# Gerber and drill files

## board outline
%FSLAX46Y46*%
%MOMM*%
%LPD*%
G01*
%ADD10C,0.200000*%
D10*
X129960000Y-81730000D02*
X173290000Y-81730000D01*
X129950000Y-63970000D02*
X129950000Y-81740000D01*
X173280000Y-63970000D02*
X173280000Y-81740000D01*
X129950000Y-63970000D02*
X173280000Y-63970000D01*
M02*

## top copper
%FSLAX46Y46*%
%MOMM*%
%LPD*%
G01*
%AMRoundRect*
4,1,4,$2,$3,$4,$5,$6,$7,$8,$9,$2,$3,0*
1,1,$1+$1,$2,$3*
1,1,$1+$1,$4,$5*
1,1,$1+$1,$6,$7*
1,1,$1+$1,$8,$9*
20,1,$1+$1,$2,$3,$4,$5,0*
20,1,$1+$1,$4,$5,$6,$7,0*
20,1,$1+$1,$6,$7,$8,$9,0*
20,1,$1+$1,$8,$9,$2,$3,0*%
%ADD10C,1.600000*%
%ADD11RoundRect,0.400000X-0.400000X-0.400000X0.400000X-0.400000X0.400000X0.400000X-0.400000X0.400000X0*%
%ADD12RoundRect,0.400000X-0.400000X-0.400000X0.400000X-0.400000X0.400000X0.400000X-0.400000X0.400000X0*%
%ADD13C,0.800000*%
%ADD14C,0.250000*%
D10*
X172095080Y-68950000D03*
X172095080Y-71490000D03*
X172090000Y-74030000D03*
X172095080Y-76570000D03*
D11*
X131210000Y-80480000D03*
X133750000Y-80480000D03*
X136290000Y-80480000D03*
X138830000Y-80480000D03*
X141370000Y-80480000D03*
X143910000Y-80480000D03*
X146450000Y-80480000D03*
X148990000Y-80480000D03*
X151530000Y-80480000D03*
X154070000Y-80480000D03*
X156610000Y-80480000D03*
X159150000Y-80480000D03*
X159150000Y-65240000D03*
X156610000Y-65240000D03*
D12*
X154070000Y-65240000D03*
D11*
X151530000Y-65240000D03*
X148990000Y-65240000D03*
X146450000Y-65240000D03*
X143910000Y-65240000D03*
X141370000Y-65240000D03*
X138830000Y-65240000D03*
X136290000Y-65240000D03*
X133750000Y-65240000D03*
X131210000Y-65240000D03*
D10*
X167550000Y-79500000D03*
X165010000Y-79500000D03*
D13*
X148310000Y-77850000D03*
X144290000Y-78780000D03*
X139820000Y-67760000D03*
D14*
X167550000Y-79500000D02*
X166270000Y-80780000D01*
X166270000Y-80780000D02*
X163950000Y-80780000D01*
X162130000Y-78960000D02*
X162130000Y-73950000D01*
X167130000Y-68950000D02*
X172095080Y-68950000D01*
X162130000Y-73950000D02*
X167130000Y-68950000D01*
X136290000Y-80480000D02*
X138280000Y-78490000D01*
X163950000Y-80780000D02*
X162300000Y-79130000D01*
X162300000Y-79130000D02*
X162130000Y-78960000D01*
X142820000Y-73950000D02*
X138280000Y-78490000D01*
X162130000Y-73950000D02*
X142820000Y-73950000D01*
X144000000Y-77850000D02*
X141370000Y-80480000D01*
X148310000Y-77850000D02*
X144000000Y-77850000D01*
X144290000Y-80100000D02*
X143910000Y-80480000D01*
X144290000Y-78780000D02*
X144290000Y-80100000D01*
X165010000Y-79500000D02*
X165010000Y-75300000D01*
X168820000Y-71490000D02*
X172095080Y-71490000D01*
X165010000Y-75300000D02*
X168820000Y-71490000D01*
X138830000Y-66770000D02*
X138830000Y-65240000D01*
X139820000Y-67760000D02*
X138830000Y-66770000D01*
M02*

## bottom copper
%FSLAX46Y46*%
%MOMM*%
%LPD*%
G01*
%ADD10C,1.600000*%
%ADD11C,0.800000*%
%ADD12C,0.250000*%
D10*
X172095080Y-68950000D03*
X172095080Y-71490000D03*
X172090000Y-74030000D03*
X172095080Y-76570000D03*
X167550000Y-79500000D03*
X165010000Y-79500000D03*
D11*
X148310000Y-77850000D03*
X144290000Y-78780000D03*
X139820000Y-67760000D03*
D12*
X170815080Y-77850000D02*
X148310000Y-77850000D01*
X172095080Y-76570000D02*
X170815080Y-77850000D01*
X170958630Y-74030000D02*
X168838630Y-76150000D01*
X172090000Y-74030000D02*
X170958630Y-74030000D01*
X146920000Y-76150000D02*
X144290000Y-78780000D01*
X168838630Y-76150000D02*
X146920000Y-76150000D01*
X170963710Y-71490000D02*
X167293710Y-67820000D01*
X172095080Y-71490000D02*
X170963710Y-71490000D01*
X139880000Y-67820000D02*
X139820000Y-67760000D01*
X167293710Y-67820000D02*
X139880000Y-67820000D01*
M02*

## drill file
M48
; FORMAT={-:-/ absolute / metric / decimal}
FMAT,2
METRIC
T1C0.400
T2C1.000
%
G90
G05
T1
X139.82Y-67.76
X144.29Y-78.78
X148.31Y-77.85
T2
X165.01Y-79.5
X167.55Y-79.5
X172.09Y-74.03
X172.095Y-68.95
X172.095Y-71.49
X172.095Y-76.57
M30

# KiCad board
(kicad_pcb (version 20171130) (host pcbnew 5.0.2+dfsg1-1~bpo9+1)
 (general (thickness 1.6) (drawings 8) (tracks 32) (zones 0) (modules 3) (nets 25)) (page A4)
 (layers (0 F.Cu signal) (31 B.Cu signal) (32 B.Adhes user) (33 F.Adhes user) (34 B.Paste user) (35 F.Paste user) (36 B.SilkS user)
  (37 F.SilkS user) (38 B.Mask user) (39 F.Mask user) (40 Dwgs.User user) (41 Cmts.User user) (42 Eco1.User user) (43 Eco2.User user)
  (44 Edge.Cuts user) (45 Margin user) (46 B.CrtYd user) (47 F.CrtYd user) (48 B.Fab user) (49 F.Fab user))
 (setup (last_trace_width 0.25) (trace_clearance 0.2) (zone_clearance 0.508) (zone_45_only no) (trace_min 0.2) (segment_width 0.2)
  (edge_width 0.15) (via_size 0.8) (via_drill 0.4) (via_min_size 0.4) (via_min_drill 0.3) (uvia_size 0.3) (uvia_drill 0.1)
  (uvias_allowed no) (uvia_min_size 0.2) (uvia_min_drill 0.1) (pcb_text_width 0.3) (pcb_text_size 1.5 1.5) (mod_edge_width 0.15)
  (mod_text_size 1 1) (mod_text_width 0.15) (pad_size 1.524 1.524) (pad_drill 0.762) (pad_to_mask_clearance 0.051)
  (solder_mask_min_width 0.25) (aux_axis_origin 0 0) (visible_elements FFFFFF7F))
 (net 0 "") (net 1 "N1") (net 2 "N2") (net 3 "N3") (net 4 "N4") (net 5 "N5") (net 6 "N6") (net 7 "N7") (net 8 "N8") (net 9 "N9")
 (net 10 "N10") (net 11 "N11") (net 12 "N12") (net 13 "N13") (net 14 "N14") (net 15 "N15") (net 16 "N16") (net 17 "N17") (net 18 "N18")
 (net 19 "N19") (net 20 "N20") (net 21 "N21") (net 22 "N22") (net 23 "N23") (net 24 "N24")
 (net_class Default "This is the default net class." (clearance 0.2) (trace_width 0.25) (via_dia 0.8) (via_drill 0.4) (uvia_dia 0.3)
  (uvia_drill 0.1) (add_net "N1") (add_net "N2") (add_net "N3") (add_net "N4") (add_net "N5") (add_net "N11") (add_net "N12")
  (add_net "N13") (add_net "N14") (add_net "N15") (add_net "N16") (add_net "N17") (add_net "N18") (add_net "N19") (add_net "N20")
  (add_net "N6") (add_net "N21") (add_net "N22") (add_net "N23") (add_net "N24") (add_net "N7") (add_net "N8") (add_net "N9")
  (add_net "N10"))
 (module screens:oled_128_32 (layer F.Cu) (at 172.09508 72.76 270)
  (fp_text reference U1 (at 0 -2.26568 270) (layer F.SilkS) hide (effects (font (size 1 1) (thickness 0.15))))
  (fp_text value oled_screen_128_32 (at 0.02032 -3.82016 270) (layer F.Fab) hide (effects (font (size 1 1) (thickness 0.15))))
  (pad 1 thru_hole circle (at -3.81 0 270) (size 1.6 1.6) (drill 1) (layers *.Cu *.Mask) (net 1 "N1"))
  (pad 2 thru_hole circle (at -1.27 0 270) (size 1.6 1.6) (drill 1) (layers *.Cu *.Mask) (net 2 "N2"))
  (pad 3 thru_hole circle (at 1.27 0.00508 270) (size 1.6 1.6) (drill 1) (layers *.Cu *.Mask) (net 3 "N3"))
  (pad 4 thru_hole circle (at 3.81 0 270) (size 1.6 1.6) (drill 1) (layers *.Cu *.Mask) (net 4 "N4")))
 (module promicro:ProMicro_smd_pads (layer F.Cu) (at 145.18 72.86)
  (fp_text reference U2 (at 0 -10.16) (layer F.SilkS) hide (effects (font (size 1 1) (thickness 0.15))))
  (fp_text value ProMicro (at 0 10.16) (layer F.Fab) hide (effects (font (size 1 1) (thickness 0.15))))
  (pad 1 smd roundrect (at -13.97 7.62) (size 1.6 1.6) (layers F.Cu F.Paste F.Mask) (roundrect_rratio 0.25) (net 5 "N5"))
  (pad 2 smd roundrect (at -11.43 7.62) (size 1.6 1.6) (layers F.Cu F.Paste F.Mask) (roundrect_rratio 0.25) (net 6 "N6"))
  (pad 3 smd roundrect (at -8.89 7.62) (size 1.6 1.6) (layers F.Cu F.Paste F.Mask) (roundrect_rratio 0.25) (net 1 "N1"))
  (pad 4 smd roundrect (at -6.35 7.62) (size 1.6 1.6) (layers F.Cu F.Paste F.Mask) (roundrect_rratio 0.25) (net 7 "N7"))
  (pad 5 smd roundrect (at -3.81 7.62) (size 1.6 1.6) (layers F.Cu F.Paste F.Mask) (roundrect_rratio 0.25) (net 4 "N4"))
  (pad 6 smd roundrect (at -1.27 7.62) (size 1.6 1.6) (layers F.Cu F.Paste F.Mask) (roundrect_rratio 0.25) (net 3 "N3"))
  (pad 7 smd roundrect (at 1.27 7.62) (size 1.6 1.6) (layers F.Cu F.Paste F.Mask) (roundrect_rratio 0.25) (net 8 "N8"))
  (pad 8 smd roundrect (at 3.81 7.62) (size 1.6 1.6) (layers F.Cu F.Paste F.Mask) (roundrect_rratio 0.25) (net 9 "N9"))
  (pad 9 smd roundrect (at 6.35 7.62) (size 1.6 1.6) (layers F.Cu F.Paste F.Mask) (roundrect_rratio 0.25) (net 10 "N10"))
  (pad 10 smd roundrect (at 8.89 7.62) (size 1.6 1.6) (layers F.Cu F.Paste F.Mask) (roundrect_rratio 0.25) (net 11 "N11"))
  (pad 11 smd roundrect (at 11.43 7.62) (size 1.6 1.6) (layers F.Cu F.Paste F.Mask) (roundrect_rratio 0.25) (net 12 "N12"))
  (pad 12 smd roundrect (at 13.97 7.62) (size 1.6 1.6) (layers F.Cu F.Paste F.Mask) (roundrect_rratio 0.25) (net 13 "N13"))
  (pad 13 smd roundrect (at 13.97 -7.62) (size 1.6 1.6) (layers F.Cu F.Paste F.Mask) (roundrect_rratio 0.25) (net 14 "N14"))
  (pad 14 smd roundrect (at 11.43 -7.62) (size 1.6 1.6) (layers F.Cu F.Paste F.Mask) (roundrect_rratio 0.25) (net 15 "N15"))
  (pad 15 connect roundrect (at 8.89 -7.62) (size 1.6 1.6) (layers F.Cu F.Mask) (roundrect_rratio 0.25) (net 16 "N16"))
  (pad 16 smd roundrect (at 6.35 -7.62) (size 1.6 1.6) (layers F.Cu F.Paste F.Mask) (roundrect_rratio 0.25) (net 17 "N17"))
  (pad 17 smd roundrect (at 3.81 -7.62) (size 1.6 1.6) (layers F.Cu F.Paste F.Mask) (roundrect_rratio 0.25) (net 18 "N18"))
  (pad 18 smd roundrect (at 1.27 -7.62) (size 1.6 1.6) (layers F.Cu F.Paste F.Mask) (roundrect_rratio 0.25) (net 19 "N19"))
  (pad 19 smd roundrect (at -1.27 -7.62) (size 1.6 1.6) (layers F.Cu F.Paste F.Mask) (roundrect_rratio 0.25) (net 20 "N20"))
  (pad 20 smd roundrect (at -3.81 -7.62) (size 1.6 1.6) (layers F.Cu F.Paste F.Mask) (roundrect_rratio 0.25) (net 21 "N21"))
  (pad 21 smd roundrect (at -6.35 -7.62) (size 1.6 1.6) (layers F.Cu F.Paste F.Mask) (roundrect_rratio 0.25) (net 2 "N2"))
  (pad 22 smd roundrect (at -8.89 -7.62) (size 1.6 1.6) (layers F.Cu F.Paste F.Mask) (roundrect_rratio 0.25) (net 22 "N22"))
  (pad 23 smd roundrect (at -11.43 -7.62) (size 1.6 1.6) (layers F.Cu F.Paste F.Mask) (roundrect_rratio 0.25) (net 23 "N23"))
  (pad 24 smd roundrect (at -13.97 -7.62) (size 1.6 1.6) (layers F.Cu F.Paste F.Mask) (roundrect_rratio 0.25) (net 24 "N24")))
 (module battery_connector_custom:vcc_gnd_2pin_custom (layer F.Cu) (at 166.28 79.5 180)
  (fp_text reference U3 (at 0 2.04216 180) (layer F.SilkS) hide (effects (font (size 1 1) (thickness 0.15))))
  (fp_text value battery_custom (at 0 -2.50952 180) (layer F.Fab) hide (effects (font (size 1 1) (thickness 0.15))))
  (pad 1 thru_hole circle (at -1.27 0 180) (size 1.6 1.6) (drill 1) (layers *.Cu *.Mask) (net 1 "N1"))
  (pad 2 thru_hole circle (at 1.27 0 180) (size 1.6 1.6) (drill 1) (layers *.Cu *.Mask) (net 2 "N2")))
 (gr_line (start 129.96 81.73) (end 173.29 81.73) (layer Edge.Cuts) (width 0.2))
 (gr_line (start 129.95 63.97) (end 129.95 81.74) (layer Edge.Cuts) (width 0.2))
 (gr_line (start 173.28 63.97) (end 173.28 81.74) (layer Edge.Cuts) (width 0.2))
 (gr_line (start 129.95 63.97) (end 173.28 63.97) (layer Edge.Cuts) (width 0.2))
 (segment (start 167.55 79.5) (end 166.27 80.78) (width 0.25) (layer F.Cu) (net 1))
 (segment (start 166.27 80.78) (end 163.95 80.78) (width 0.25) (layer F.Cu) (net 1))
 (segment (start 162.13 78.96) (end 162.13 73.95) (width 0.25) (layer F.Cu) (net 1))
 (segment (start 167.13 68.95) (end 172.09508 68.95) (width 0.25) (layer F.Cu) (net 1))
 (segment (start 162.13 73.95) (end 167.13 68.95) (width 0.25) (layer F.Cu) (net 1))
 (segment (start 136.29 80.48) (end 138.28 78.49) (width 0.25) (layer F.Cu) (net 1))
 (segment (start 163.95 80.78) (end 162.3 79.13) (width 0.25) (layer F.Cu) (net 1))
 (segment (start 162.3 79.13) (end 162.13 78.96) (width 0.25) (layer F.Cu) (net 1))
 (segment (start 142.82 73.95) (end 138.28 78.49) (width 0.25) (layer F.Cu) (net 1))
 (segment (start 162.13 73.95) (end 142.82 73.95) (width 0.25) (layer F.Cu) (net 1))
 (via (at 148.31 77.85) (size 0.8) (drill 0.4) (layers F.Cu B.Cu) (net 4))
 (segment (start 170.81508 77.85) (end 148.31 77.85) (width 0.25) (layer B.Cu) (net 4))
 (segment (start 172.09508 76.57) (end 170.81508 77.85) (width 0.25) (layer B.Cu) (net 4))
 (segment (start 144 77.85) (end 141.37 80.48) (width 0.25) (layer F.Cu) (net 4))
 (segment (start 148.31 77.85) (end 144 77.85) (width 0.25) (layer F.Cu) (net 4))
 (segment (start 170.95863 74.03) (end 168.83863 76.15) (width 0.25) (layer B.Cu) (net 3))
 (segment (start 172.09 74.03) (end 170.95863 74.03) (width 0.25) (layer B.Cu) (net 3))
 (via (at 144.29 78.78) (size 0.8) (drill 0.4) (layers F.Cu B.Cu) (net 3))
 (segment (start 146.92 76.15) (end 144.29 78.78) (width 0.25) (layer B.Cu) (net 3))
 (segment (start 168.83863 76.15) (end 146.92 76.15) (width 0.25) (layer B.Cu) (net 3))
 (segment (start 144.29 80.1) (end 143.91 80.48) (width 0.25) (layer F.Cu) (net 3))
 (segment (start 144.29 78.78) (end 144.29 80.1) (width 0.25) (layer F.Cu) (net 3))
 (segment (start 165.01 79.5) (end 165.01 75.3) (width 0.25) (layer F.Cu) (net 2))
 (segment (start 168.82 71.49) (end 172.09508 71.49) (width 0.25) (layer F.Cu) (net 2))
 (segment (start 165.01 75.3) (end 168.82 71.49) (width 0.25) (layer F.Cu) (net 2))
 (segment (start 170.96371 71.49) (end 167.29371 67.82) (width 0.25) (layer B.Cu) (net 2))
 (segment (start 172.09508 71.49) (end 170.96371 71.49) (width 0.25) (layer B.Cu) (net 2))
 (via (at 139.82 67.76) (size 0.8) (drill 0.4) (layers F.Cu B.Cu) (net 2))
 (segment (start 139.88 67.82) (end 139.82 67.76) (width 0.25) (layer B.Cu) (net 2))
 (segment (start 167.29371 67.82) (end 139.88 67.82) (width 0.25) (layer B.Cu) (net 2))
 (segment (start 138.83 66.77) (end 138.83 65.24) (width 0.25) (layer F.Cu) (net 2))
 (segment (start 139.82 67.76) (end 138.83 66.77) (width 0.25) (layer F.Cu) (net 2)))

